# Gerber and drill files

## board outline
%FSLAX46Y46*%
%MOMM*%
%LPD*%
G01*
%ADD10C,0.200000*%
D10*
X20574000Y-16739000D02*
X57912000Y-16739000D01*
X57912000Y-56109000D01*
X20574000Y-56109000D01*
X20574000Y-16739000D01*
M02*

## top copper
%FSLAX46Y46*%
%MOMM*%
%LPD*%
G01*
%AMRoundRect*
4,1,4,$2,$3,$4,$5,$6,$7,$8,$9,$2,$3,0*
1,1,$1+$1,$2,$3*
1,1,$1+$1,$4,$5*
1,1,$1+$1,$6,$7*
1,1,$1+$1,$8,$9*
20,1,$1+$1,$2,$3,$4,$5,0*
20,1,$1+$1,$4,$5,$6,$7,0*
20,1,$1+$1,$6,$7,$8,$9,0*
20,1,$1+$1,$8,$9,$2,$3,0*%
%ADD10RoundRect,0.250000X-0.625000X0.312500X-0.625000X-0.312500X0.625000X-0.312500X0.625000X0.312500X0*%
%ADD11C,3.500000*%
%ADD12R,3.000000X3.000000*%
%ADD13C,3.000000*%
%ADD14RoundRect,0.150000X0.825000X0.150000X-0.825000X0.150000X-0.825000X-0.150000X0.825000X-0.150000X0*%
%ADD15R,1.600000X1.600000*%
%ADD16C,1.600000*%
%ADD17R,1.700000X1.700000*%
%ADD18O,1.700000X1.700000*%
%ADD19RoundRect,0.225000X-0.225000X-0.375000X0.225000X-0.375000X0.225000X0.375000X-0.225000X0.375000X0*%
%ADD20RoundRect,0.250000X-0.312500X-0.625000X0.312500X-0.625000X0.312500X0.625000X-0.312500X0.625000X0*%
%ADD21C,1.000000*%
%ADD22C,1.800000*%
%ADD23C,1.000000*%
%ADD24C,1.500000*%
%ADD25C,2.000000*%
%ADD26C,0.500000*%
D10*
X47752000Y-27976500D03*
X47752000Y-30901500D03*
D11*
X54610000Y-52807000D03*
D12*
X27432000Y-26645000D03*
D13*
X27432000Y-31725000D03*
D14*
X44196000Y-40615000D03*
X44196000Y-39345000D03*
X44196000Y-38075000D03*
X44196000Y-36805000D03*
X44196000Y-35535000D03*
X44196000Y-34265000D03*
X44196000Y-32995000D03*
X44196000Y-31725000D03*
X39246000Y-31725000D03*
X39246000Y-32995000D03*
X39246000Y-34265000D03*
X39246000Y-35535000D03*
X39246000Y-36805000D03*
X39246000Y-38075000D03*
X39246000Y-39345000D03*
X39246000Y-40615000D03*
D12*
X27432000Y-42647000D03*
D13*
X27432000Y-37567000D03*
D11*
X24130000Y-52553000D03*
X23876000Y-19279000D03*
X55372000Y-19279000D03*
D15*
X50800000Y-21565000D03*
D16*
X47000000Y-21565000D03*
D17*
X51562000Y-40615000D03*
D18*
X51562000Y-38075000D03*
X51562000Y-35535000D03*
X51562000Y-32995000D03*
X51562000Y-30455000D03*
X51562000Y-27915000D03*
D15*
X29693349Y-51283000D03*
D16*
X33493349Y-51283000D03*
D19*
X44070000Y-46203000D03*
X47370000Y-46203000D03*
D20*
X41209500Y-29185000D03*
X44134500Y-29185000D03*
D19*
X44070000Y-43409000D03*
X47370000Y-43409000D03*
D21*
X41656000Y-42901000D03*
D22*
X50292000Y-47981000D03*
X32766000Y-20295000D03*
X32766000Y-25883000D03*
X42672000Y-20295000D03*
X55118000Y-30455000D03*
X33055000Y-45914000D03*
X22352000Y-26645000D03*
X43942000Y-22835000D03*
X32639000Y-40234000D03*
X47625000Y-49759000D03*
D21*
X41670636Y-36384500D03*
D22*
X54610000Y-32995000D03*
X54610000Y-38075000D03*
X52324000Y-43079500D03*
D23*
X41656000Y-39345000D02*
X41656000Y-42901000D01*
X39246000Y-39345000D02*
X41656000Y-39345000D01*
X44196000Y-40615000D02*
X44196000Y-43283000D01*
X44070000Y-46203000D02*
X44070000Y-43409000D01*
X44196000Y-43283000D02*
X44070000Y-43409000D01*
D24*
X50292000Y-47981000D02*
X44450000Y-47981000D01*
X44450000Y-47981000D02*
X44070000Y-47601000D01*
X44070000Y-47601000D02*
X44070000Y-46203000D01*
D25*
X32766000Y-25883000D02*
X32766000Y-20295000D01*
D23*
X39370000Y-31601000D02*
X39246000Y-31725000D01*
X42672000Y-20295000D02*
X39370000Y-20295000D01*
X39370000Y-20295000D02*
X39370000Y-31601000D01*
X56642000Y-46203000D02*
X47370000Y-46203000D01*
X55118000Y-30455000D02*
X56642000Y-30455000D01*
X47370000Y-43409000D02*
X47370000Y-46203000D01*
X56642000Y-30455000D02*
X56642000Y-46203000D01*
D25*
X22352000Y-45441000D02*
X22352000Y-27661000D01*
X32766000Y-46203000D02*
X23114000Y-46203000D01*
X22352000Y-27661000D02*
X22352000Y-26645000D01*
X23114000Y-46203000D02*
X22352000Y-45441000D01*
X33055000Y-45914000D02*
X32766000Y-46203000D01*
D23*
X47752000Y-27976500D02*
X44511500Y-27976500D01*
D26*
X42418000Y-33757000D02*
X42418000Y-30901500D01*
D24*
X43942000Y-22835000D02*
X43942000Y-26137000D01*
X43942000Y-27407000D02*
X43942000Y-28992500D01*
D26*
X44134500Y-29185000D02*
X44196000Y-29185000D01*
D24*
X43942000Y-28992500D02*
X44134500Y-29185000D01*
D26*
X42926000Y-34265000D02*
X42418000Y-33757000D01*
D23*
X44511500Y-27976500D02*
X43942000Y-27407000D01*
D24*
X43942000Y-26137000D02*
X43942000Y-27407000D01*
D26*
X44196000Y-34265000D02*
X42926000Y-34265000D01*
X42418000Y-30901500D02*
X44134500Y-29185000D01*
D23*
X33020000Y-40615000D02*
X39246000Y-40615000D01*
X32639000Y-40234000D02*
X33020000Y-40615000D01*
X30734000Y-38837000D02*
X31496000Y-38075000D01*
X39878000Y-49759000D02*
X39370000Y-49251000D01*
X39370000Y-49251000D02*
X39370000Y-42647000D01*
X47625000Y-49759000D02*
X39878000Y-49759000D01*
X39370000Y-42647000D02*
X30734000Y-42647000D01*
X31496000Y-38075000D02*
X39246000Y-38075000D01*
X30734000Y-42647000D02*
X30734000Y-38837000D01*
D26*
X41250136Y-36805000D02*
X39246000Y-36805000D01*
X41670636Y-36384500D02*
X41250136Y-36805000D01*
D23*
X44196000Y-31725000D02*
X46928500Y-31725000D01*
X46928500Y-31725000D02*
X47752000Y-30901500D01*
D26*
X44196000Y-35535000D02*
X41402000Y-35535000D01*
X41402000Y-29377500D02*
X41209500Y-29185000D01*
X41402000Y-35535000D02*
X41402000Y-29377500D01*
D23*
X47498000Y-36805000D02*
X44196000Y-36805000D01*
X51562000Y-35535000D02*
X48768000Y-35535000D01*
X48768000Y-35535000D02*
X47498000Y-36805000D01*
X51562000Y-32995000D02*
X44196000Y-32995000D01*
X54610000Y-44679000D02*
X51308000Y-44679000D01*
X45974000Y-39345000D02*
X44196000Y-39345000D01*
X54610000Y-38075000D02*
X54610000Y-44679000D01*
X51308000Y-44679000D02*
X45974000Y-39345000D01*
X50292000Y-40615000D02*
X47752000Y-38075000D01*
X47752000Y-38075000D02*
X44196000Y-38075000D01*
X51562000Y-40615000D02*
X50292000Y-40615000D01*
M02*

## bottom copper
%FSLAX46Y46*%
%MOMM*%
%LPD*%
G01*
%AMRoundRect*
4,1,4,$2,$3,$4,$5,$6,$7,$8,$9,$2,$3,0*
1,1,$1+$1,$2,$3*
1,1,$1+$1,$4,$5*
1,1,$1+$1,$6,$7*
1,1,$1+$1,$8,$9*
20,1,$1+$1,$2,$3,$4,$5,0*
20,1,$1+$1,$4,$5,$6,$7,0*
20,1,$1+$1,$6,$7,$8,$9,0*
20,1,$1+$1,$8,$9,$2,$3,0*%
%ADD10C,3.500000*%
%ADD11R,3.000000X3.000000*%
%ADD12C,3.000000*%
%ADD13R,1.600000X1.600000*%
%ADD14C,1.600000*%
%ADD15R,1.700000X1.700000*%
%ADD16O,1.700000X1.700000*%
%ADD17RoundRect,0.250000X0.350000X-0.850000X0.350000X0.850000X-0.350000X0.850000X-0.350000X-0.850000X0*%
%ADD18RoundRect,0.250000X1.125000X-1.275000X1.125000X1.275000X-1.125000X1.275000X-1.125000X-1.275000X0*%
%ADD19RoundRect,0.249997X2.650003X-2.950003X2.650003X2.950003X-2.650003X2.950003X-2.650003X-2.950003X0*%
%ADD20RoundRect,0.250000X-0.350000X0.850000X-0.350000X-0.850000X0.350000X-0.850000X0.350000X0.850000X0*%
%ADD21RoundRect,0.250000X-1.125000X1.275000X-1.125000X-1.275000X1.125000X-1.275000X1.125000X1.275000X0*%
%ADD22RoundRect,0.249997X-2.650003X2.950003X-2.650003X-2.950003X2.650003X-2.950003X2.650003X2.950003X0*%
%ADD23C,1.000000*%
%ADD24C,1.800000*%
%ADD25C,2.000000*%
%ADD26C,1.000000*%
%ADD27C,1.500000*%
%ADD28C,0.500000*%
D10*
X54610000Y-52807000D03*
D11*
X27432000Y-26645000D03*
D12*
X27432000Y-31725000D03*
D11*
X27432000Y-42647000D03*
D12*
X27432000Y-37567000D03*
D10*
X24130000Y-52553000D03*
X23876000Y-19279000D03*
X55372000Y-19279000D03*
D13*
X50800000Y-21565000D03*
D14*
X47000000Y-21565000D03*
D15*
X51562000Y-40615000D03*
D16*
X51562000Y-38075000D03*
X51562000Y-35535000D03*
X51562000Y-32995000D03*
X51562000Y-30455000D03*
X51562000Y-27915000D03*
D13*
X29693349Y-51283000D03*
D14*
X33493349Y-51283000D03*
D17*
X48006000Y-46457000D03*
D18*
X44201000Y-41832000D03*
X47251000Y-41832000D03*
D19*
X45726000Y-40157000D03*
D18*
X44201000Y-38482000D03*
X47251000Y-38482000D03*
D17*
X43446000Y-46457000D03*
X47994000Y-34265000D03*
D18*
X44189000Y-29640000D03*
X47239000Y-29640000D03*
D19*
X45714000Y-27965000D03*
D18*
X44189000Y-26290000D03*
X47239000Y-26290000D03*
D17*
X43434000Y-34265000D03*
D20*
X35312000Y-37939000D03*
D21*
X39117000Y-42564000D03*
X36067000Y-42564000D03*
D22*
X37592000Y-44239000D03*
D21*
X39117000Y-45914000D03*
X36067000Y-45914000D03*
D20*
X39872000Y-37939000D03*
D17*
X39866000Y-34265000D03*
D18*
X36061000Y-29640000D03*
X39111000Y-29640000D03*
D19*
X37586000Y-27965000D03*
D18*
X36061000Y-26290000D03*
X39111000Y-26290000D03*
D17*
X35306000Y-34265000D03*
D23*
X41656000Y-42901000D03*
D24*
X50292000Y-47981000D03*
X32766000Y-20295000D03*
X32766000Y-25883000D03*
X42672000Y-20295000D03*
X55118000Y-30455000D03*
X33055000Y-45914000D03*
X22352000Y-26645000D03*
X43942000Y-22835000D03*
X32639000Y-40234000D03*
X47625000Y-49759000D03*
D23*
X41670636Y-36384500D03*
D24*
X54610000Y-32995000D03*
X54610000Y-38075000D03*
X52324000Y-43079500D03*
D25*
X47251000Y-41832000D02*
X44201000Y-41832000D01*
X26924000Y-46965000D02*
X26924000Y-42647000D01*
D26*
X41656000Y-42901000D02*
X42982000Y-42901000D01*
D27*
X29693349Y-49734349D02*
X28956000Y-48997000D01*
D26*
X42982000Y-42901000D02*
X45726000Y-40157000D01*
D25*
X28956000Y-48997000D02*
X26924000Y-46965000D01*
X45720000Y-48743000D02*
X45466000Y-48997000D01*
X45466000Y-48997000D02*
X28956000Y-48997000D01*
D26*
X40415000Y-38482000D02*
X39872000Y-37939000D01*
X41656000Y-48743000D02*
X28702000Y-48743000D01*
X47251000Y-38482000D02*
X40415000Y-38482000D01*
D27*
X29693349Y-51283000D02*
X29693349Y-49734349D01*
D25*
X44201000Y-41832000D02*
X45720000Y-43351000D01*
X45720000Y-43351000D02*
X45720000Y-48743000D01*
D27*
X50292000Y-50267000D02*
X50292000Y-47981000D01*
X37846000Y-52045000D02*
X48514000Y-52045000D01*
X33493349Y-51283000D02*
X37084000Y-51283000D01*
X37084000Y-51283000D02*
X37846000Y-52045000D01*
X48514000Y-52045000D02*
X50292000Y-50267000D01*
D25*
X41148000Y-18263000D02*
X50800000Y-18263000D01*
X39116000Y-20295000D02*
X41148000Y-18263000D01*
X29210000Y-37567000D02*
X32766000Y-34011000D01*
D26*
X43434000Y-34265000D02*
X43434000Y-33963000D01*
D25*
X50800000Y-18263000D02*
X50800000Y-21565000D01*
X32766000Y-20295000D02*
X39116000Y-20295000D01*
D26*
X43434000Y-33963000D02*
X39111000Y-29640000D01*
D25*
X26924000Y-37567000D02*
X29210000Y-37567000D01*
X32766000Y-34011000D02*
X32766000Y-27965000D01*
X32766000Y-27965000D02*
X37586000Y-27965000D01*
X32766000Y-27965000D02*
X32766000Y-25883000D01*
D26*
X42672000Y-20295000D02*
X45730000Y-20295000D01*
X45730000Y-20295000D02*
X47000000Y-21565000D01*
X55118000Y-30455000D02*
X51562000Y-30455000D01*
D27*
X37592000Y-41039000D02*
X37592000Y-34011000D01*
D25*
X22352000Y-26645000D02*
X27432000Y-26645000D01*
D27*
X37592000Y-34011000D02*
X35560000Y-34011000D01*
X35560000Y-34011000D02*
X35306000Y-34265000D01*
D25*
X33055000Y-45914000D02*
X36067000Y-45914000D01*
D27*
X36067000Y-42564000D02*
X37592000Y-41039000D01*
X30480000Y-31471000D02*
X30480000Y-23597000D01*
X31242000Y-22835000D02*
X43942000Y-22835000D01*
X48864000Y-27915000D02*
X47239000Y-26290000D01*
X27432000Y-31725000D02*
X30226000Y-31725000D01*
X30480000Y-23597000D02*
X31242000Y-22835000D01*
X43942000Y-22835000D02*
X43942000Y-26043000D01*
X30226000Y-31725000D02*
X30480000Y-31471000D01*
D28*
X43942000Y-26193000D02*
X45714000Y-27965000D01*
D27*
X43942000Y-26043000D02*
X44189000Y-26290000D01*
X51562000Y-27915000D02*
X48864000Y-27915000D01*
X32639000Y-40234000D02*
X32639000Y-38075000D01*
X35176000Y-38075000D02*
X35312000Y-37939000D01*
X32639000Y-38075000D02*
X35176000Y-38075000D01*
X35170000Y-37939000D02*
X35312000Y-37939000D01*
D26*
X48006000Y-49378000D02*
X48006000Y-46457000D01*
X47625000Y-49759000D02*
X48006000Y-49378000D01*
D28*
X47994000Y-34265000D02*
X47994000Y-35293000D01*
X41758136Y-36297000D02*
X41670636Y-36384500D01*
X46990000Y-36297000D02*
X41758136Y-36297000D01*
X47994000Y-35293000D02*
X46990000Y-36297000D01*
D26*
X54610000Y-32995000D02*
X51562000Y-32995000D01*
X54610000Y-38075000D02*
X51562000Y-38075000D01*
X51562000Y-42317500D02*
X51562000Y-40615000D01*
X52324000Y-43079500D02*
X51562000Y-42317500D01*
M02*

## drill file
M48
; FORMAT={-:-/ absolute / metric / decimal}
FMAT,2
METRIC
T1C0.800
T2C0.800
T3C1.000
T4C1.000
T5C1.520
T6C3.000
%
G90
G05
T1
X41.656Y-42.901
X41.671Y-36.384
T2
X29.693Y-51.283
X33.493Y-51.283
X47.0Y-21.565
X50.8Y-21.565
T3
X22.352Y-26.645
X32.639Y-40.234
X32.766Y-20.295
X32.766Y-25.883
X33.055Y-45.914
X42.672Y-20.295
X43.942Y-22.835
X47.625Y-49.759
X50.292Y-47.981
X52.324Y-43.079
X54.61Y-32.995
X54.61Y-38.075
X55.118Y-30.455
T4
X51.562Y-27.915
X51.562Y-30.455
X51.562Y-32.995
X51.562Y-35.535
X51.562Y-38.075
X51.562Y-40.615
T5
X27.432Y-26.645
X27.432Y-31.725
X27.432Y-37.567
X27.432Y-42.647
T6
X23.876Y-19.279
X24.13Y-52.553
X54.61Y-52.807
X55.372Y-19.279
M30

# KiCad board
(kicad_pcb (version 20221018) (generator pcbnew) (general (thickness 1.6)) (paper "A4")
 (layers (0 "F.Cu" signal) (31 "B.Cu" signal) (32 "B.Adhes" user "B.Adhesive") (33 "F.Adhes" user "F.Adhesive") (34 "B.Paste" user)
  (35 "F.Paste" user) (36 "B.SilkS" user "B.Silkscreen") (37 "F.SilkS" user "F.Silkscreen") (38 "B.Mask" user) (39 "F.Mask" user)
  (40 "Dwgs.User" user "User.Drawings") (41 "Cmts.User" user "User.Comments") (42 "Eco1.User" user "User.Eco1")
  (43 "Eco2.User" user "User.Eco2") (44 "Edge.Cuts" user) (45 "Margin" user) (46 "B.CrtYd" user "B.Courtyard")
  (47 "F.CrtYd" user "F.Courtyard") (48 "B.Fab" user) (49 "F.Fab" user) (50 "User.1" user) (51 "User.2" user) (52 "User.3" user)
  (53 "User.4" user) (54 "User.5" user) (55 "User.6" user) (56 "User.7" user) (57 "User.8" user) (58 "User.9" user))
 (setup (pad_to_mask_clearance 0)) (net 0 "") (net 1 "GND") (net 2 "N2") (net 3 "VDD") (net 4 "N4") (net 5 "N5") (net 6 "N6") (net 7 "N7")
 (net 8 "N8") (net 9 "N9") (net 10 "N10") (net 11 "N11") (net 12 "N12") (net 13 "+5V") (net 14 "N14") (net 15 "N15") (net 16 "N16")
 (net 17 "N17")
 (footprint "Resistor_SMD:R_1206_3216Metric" (layer "F.Cu") (at 47.752 29.439 -90)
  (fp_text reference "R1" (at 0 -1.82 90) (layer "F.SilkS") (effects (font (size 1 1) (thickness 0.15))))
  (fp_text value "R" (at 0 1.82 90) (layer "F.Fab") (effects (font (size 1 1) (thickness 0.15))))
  (pad "1" smd roundrect (at -1.4625 0 270) (size 1.125 1.75) (layers "F.Cu" "F.Paste" "F.Mask") (roundrect_rratio 0.222222) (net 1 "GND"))
  (pad "2" smd roundrect (at 1.4625 0 270) (size 1.125 1.75) (layers "F.Cu" "F.Paste" "F.Mask") (roundrect_rratio 0.222222) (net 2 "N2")))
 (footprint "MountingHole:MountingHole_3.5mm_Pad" (layer "F.Cu") (at 54.61 52.807)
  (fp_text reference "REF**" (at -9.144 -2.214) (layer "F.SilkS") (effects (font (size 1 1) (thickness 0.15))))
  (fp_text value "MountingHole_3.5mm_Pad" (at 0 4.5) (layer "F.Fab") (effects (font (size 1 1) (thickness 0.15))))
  (pad "1" thru_hole circle (at 0 0) (size 3.5 3.5) (drill 3) (layers "*.Cu" "*.Mask")))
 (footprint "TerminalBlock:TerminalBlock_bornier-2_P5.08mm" (layer "F.Cu") (at 27.432 26.645 -90)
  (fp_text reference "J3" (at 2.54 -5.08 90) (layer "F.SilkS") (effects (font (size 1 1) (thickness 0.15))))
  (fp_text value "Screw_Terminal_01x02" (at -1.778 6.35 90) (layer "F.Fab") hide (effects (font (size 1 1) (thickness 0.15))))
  (pad "1" thru_hole rect (at 0 0 270) (size 3 3) (drill 1.52) (layers "*.Cu" "*.Mask") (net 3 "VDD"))
  (pad "2" thru_hole circle (at 5.08 0 270) (size 3 3) (drill 1.52) (layers "*.Cu" "*.Mask") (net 1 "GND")))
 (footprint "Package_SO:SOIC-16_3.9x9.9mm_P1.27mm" (layer "F.Cu") (at 41.721 36.17 180)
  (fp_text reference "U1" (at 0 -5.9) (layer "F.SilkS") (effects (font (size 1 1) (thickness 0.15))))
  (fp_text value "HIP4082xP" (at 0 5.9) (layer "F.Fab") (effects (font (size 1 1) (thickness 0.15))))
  (pad "1" smd roundrect (at -2.475 -4.445 180) (size 1.95 0.6) (layers "F.Cu" "F.Paste" "F.Mask") (roundrect_rratio 0.25) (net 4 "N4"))
  (pad "2" smd roundrect (at -2.475 -3.175 180) (size 1.95 0.6) (layers "F.Cu" "F.Paste" "F.Mask") (roundrect_rratio 0.25) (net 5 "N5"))
  (pad "3" smd roundrect (at -2.475 -1.905 180) (size 1.95 0.6) (layers "F.Cu" "F.Paste" "F.Mask") (roundrect_rratio 0.25) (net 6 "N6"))
  (pad "4" smd roundrect (at -2.475 -0.635 180) (size 1.95 0.6) (layers "F.Cu" "F.Paste" "F.Mask") (roundrect_rratio 0.25) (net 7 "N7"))
  (pad "5" smd roundrect (at -2.475 0.635 180) (size 1.95 0.6) (layers "F.Cu" "F.Paste" "F.Mask") (roundrect_rratio 0.25) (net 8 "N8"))
  (pad "6" smd roundrect (at -2.475 1.905 180) (size 1.95 0.6) (layers "F.Cu" "F.Paste" "F.Mask") (roundrect_rratio 0.25) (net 1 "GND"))
  (pad "7" smd roundrect (at -2.475 3.175 180) (size 1.95 0.6) (layers "F.Cu" "F.Paste" "F.Mask") (roundrect_rratio 0.25) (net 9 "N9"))
  (pad "8" smd roundrect (at -2.475 4.445 180) (size 1.95 0.6) (layers "F.Cu" "F.Paste" "F.Mask") (roundrect_rratio 0.25) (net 2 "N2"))
  (pad "9" smd roundrect (at 2.475 4.445 180) (size 1.95 0.6) (layers "F.Cu" "F.Paste" "F.Mask") (roundrect_rratio 0.25) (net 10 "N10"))
  (pad "10" smd roundrect (at 2.475 3.175 180) (size 1.95 0.6) (layers "F.Cu" "F.Paste" "F.Mask") (roundrect_rratio 0.25) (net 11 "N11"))
  (pad "11" smd roundrect (at 2.475 1.905 180) (size 1.95 0.6) (layers "F.Cu" "F.Paste" "F.Mask") (roundrect_rratio 0.25) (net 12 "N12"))
  (pad "12" smd roundrect (at 2.475 0.635 180) (size 1.95 0.6) (layers "F.Cu" "F.Paste" "F.Mask") (roundrect_rratio 0.25) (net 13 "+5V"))
  (pad "13" smd roundrect (at 2.475 -0.635 180) (size 1.95 0.6) (layers "F.Cu" "F.Paste" "F.Mask") (roundrect_rratio 0.25) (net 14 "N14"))
  (pad "14" smd roundrect (at 2.475 -1.905 180) (size 1.95 0.6) (layers "F.Cu" "F.Paste" "F.Mask") (roundrect_rratio 0.25) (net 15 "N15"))
  (pad "15" smd roundrect (at 2.475 -3.175 180) (size 1.95 0.6) (layers "F.Cu" "F.Paste" "F.Mask") (roundrect_rratio 0.25) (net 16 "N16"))
  (pad "16" smd roundrect (at 2.475 -4.445 180) (size 1.95 0.6) (layers "F.Cu" "F.Paste" "F.Mask") (roundrect_rratio 0.25) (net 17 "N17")))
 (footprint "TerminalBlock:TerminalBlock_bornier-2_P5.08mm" (layer "F.Cu") (at 27.432 42.647 90)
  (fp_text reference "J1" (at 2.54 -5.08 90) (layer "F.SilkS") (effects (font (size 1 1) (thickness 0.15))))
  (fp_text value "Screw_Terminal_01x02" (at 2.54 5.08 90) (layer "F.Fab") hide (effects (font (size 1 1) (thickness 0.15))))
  (pad "1" thru_hole rect (at 0 0 90) (size 3 3) (drill 1.52) (layers "*.Cu" "*.Mask") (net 16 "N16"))
  (pad "2" thru_hole circle (at 5.08 0 90) (size 3 3) (drill 1.52) (layers "*.Cu" "*.Mask") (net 12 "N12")))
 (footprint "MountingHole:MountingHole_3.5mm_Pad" (layer "F.Cu") (at 24.13 52.553)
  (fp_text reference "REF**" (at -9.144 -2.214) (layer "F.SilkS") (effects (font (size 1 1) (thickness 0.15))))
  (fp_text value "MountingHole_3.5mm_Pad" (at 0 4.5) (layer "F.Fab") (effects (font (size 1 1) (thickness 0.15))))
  (pad "1" thru_hole circle (at 0 0) (size 3.5 3.5) (drill 3) (layers "*.Cu" "*.Mask")))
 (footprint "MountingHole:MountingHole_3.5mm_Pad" (layer "F.Cu") (at 23.876 19.279)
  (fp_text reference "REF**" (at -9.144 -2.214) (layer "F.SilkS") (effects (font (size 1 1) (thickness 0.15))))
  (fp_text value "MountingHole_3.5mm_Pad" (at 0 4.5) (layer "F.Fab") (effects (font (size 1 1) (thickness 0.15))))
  (pad "1" thru_hole circle (at 0 0) (size 3.5 3.5) (drill 3) (layers "*.Cu" "*.Mask")))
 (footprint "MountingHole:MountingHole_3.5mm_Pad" (layer "F.Cu") (at 55.372 19.279)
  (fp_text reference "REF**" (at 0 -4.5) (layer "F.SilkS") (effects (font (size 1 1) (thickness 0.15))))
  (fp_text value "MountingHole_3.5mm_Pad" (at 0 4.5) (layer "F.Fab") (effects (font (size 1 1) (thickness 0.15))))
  (pad "1" thru_hole circle (at 0 0) (size 3.5 3.5) (drill 3) (layers "*.Cu" "*.Mask")))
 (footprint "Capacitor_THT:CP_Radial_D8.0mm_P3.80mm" (layer "F.Cu") (at 50.8 21.565 180)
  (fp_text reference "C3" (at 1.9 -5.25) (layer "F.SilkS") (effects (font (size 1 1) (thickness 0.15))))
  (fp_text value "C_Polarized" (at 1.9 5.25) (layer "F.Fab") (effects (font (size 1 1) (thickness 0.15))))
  (pad "1" thru_hole rect (at 0 0 180) (size 1.6 1.6) (drill 0.8) (layers "*.Cu" "*.Mask") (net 12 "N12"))
  (pad "2" thru_hole circle (at 3.8 0 180) (size 1.6 1.6) (drill 0.8) (layers "*.Cu" "*.Mask") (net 10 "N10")))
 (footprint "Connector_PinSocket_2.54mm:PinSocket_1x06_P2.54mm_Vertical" (layer "F.Cu") (at 51.562 40.615 180)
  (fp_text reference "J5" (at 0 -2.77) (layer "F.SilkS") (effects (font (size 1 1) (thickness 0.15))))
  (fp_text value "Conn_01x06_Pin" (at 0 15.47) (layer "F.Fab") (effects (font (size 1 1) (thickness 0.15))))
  (pad "1" thru_hole rect (at 0 0 180) (size 1.7 1.7) (drill 1) (layers "*.Cu" "*.Mask") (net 6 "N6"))
  (pad "2" thru_hole oval (at 0 2.54 180) (size 1.7 1.7) (drill 1) (layers "*.Cu" "*.Mask") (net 5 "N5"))
  (pad "3" thru_hole oval (at 0 5.08 180) (size 1.7 1.7) (drill 1) (layers "*.Cu" "*.Mask") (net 7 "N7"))
  (pad "4" thru_hole oval (at 0 7.62 180) (size 1.7 1.7) (drill 1) (layers "*.Cu" "*.Mask") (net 9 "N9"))
  (pad "5" thru_hole oval (at 0 10.16 180) (size 1.7 1.7) (drill 1) (layers "*.Cu" "*.Mask") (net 13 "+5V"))
  (pad "6" thru_hole oval (at 0 12.7 180) (size 1.7 1.7) (drill 1) (layers "*.Cu" "*.Mask") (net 1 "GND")))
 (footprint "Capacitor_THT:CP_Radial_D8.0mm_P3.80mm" (layer "F.Cu") (at 29.693349 51.283)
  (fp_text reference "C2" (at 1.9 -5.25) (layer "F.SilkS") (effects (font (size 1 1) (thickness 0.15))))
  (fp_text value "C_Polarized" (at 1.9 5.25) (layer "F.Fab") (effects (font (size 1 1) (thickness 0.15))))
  (pad "1" thru_hole rect (at 0 0) (size 1.6 1.6) (drill 0.8) (layers "*.Cu" "*.Mask") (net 16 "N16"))
  (pad "2" thru_hole circle (at 3.8 0) (size 1.6 1.6) (drill 0.8) (layers "*.Cu" "*.Mask") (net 4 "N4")))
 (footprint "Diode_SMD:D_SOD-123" (layer "F.Cu") (at 45.72 46.203)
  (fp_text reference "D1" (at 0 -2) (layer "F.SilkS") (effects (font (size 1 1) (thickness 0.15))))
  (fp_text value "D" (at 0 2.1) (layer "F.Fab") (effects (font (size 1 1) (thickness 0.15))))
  (pad "1" smd roundrect (at -1.65 0) (size 0.9 1.2) (layers "F.Cu" "F.Paste" "F.Mask") (roundrect_rratio 0.25) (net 4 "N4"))
  (pad "2" smd roundrect (at 1.65 0) (size 0.9 1.2) (layers "F.Cu" "F.Paste" "F.Mask") (roundrect_rratio 0.25) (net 13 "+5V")))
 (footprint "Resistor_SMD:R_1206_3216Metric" (layer "F.Cu") (at 42.672 29.185)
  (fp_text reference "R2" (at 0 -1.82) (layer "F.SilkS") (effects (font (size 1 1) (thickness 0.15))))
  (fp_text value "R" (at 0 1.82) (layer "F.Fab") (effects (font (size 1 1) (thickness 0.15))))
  (pad "1" smd roundrect (at -1.4625 0) (size 1.125 1.75) (layers "F.Cu" "F.Paste" "F.Mask") (roundrect_rratio 0.222222) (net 8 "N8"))
  (pad "2" smd roundrect (at 1.4625 0) (size 1.125 1.75) (layers "F.Cu" "F.Paste" "F.Mask") (roundrect_rratio 0.222222) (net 1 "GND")))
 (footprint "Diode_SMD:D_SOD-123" (layer "F.Cu") (at 45.72 43.409)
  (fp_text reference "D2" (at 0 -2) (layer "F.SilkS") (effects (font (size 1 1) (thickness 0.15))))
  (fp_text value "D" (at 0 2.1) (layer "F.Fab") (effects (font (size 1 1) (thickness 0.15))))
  (pad "1" smd roundrect (at -1.65 0) (size 0.9 1.2) (layers "F.Cu" "F.Paste" "F.Mask") (roundrect_rratio 0.25) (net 4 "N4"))
  (pad "2" smd roundrect (at 1.65 0) (size 0.9 1.2) (layers "F.Cu" "F.Paste" "F.Mask") (roundrect_rratio 0.25) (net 13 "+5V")))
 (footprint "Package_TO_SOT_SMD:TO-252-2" (layer "B.Cu") (at 45.726 41.417 90)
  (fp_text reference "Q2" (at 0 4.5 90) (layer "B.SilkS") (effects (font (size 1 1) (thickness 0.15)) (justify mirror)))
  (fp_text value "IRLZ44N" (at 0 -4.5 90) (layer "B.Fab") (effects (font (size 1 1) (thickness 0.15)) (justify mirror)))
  (pad "1" smd roundrect (at -5.04 2.28 90) (size 2.2 1.2) (layers "B.Cu" "B.Paste" "B.Mask") (roundrect_rratio 0.208333) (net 15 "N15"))
  (pad "2" smd roundrect (at -0.415 -1.525 90) (size 3.05 2.75) (layers "B.Cu" "B.Paste") (roundrect_rratio 0.090909) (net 16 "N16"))
  (pad "2" smd roundrect (at -0.415 1.525 90) (size 3.05 2.75) (layers "B.Cu" "B.Paste") (roundrect_rratio 0.090909) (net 16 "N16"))
  (pad "2" smd roundrect (at 1.26 0 90) (size 6.4 5.8) (layers "B.Cu" "B.Mask") (roundrect_rratio 0.043103) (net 16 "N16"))
  (pad "2" smd roundrect (at 2.935 -1.525 90) (size 3.05 2.75) (layers "B.Cu" "B.Paste") (roundrect_rratio 0.090909) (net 16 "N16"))
  (pad "2" smd roundrect (at 2.935 1.525 90) (size 3.05 2.75) (layers "B.Cu" "B.Paste") (roundrect_rratio 0.090909) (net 16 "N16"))
  (pad "3" smd roundrect (at -5.04 -2.28 90) (size 2.2 1.2) (layers "B.Cu" "B.Paste" "B.Mask") (roundrect_rratio 0.208333) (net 1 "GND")))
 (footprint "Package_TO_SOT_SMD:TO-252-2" (layer "B.Cu") (at 45.714 29.225 90)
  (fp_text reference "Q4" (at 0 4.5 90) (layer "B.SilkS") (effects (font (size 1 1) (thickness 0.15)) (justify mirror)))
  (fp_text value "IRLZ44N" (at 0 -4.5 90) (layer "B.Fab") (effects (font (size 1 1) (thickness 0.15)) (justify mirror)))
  (pad "1" smd roundrect (at -5.04 2.28 90) (size 2.2 1.2) (layers "B.Cu" "B.Paste" "B.Mask") (roundrect_rratio 0.208333) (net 14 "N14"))
  (pad "2" smd roundrect (at -0.415 -1.525 90) (size 3.05 2.75) (layers "B.Cu" "B.Paste") (roundrect_rratio 0.090909) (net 1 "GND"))
  (pad "2" smd roundrect (at -0.415 1.525 90) (size 3.05 2.75) (layers "B.Cu" "B.Paste") (roundrect_rratio 0.090909) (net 1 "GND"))
  (pad "2" smd roundrect (at 1.26 0 90) (size 6.4 5.8) (layers "B.Cu" "B.Mask") (roundrect_rratio 0.043103) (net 1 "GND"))
  (pad "2" smd roundrect (at 2.935 -1.525 90) (size 3.05 2.75) (layers "B.Cu" "B.Paste") (roundrect_rratio 0.090909) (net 1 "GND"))
  (pad "2" smd roundrect (at 2.935 1.525 90) (size 3.05 2.75) (layers "B.Cu" "B.Paste") (roundrect_rratio 0.090909) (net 1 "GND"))
  (pad "3" smd roundrect (at -5.04 -2.28 90) (size 2.2 1.2) (layers "B.Cu" "B.Paste" "B.Mask") (roundrect_rratio 0.208333) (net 12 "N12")))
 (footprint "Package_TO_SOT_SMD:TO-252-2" (layer "B.Cu") (at 37.592 42.979 -90)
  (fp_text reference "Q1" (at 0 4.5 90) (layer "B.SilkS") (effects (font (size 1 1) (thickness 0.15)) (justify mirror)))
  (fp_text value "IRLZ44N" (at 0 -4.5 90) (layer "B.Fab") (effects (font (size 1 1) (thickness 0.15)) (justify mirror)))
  (pad "1" smd roundrect (at -5.04 2.28 270) (size 2.2 1.2) (layers "B.Cu" "B.Paste" "B.Mask") (roundrect_rratio 0.208333) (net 17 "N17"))
  (pad "2" smd roundrect (at -0.415 -1.525 270) (size 3.05 2.75) (layers "B.Cu" "B.Paste") (roundrect_rratio 0.090909) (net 3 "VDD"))
  (pad "2" smd roundrect (at -0.415 1.525 270) (size 3.05 2.75) (layers "B.Cu" "B.Paste") (roundrect_rratio 0.090909) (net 3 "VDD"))
  (pad "2" smd roundrect (at 1.26 0 270) (size 6.4 5.8) (layers "B.Cu" "B.Mask") (roundrect_rratio 0.043103) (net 3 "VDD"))
  (pad "2" smd roundrect (at 2.935 -1.525 270) (size 3.05 2.75) (layers "B.Cu" "B.Paste") (roundrect_rratio 0.090909) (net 3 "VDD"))
  (pad "2" smd roundrect (at 2.935 1.525 270) (size 3.05 2.75) (layers "B.Cu" "B.Paste") (roundrect_rratio 0.090909) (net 3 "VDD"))
  (pad "3" smd roundrect (at -5.04 -2.28 270) (size 2.2 1.2) (layers "B.Cu" "B.Paste" "B.Mask") (roundrect_rratio 0.208333) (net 16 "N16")))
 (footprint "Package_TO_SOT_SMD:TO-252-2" (layer "B.Cu") (at 37.586 29.225 90)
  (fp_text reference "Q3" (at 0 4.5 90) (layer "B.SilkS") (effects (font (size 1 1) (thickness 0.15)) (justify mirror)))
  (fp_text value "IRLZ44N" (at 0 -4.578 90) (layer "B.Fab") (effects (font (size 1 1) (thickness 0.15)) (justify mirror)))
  (pad "1" smd roundrect (at -5.04 2.28 90) (size 2.2 1.2) (layers "B.Cu" "B.Paste" "B.Mask") (roundrect_rratio 0.208333) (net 11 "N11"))
  (pad "2" smd roundrect (at -0.415 -1.525 90) (size 3.05 2.75) (layers "B.Cu" "B.Paste") (roundrect_rratio 0.090909) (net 12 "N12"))
  (pad "2" smd roundrect (at -0.415 1.525 90) (size 3.05 2.75) (layers "B.Cu" "B.Paste") (roundrect_rratio 0.090909) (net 12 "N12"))
  (pad "2" smd roundrect (at 1.26 0 90) (size 6.4 5.8) (layers "B.Cu" "B.Mask") (roundrect_rratio 0.043103) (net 12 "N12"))
  (pad "2" smd roundrect (at 2.935 -1.525 90) (size 3.05 2.75) (layers "B.Cu" "B.Paste") (roundrect_rratio 0.090909) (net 12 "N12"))
  (pad "2" smd roundrect (at 2.935 1.525 90) (size 3.05 2.75) (layers "B.Cu" "B.Paste") (roundrect_rratio 0.090909) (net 12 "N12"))
  (pad "3" smd roundrect (at -5.04 -2.28 90) (size 2.2 1.2) (layers "B.Cu" "B.Paste" "B.Mask") (roundrect_rratio 0.208333) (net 3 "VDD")))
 (gr_rect (start 20.574 16.739) (end 57.912 56.109) (stroke (width 0.2) (type default)) (fill none) (layer "Edge.Cuts"))
 (segment (start 41.656 39.345) (end 41.656 42.901) (width 1) (layer "F.Cu") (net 16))
 (segment (start 39.246 39.345) (end 41.656 39.345) (width 1) (layer "F.Cu") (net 16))
 (via (at 41.656 42.901) (size 1) (drill 0.8) (layers "F.Cu" "B.Cu") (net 16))
 (segment (start 47.251 41.832) (end 44.201 41.832) (width 2) (layer "B.Cu") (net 16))
 (segment (start 26.924 46.965) (end 26.924 42.647) (width 2) (layer "B.Cu") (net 16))
 (segment (start 41.656 42.901) (end 42.982 42.901) (width 1) (layer "B.Cu") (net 16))
 (segment (start 29.693349 49.734349) (end 28.956 48.997) (width 1.5) (layer "B.Cu") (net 16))
 (segment (start 42.982 42.901) (end 45.726 40.157) (width 1) (layer "B.Cu") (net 16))
 (segment (start 28.956 48.997) (end 26.924 46.965) (width 2) (layer "B.Cu") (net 16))
 (segment (start 45.72 48.743) (end 45.466 48.997) (width 2) (layer "B.Cu") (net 16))
 (segment (start 45.466 48.997) (end 28.956 48.997) (width 2) (layer "B.Cu") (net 16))
 (segment (start 40.415 38.482) (end 39.872 37.939) (width 1) (layer "B.Cu") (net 16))
 (segment (start 41.656 48.743) (end 28.702 48.743) (width 1) (layer "B.Cu") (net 16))
 (segment (start 47.251 38.482) (end 40.415 38.482) (width 1) (layer "B.Cu") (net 16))
 (segment (start 29.693349 51.283) (end 29.693349 49.734349) (width 1.5) (layer "B.Cu") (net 16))
 (segment (start 44.201 41.832) (end 45.72 43.351) (width 2) (layer "B.Cu") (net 16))
 (segment (start 45.72 43.351) (end 45.72 48.743) (width 2) (layer "B.Cu") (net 16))
 (segment (start 44.196 40.615) (end 44.196 43.283) (width 1) (layer "F.Cu") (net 4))
 (segment (start 44.07 46.203) (end 44.07 43.409) (width 1) (layer "F.Cu") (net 4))
 (segment (start 44.196 43.283) (end 44.07 43.409) (width 1) (layer "F.Cu") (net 4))
 (segment (start 50.292 47.981) (end 44.45 47.981) (width 1.5) (layer "F.Cu") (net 4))
 (segment (start 44.45 47.981) (end 44.07 47.601) (width 1.5) (layer "F.Cu") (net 4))
 (segment (start 44.07 47.601) (end 44.07 46.203) (width 1.5) (layer "F.Cu") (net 4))
 (via (at 50.292 47.981) (size 1.8) (drill 1) (layers "F.Cu" "B.Cu") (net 4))
 (segment (start 50.292 50.267) (end 50.292 47.981) (width 1.5) (layer "B.Cu") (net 4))
 (segment (start 37.846 52.045) (end 48.514 52.045) (width 1.5) (layer "B.Cu") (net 4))
 (segment (start 33.493349 51.283) (end 37.084 51.283) (width 1.5) (layer "B.Cu") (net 4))
 (segment (start 37.084 51.283) (end 37.846 52.045) (width 1.5) (layer "B.Cu") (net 4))
 (segment (start 48.514 52.045) (end 50.292 50.267) (width 1.5) (layer "B.Cu") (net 4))
 (segment (start 32.766 25.883) (end 32.766 20.295) (width 2) (layer "F.Cu") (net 12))
 (via (at 32.766 20.295) (size 1.8) (drill 1) (layers "F.Cu" "B.Cu") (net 12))
 (via (at 32.766 25.883) (size 1.8) (drill 1) (layers "F.Cu" "B.Cu") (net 12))
 (segment (start 41.148 18.263) (end 50.8 18.263) (width 2) (layer "B.Cu") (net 12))
 (segment (start 39.116 20.295) (end 41.148 18.263) (width 2) (layer "B.Cu") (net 12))
 (segment (start 29.21 37.567) (end 32.766 34.011) (width 2) (layer "B.Cu") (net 12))
 (segment (start 43.434 34.265) (end 43.434 33.963) (width 1) (layer "B.Cu") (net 12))
 (segment (start 50.8 18.263) (end 50.8 21.565) (width 2) (layer "B.Cu") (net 12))
 (segment (start 32.766 20.295) (end 39.116 20.295) (width 2) (layer "B.Cu") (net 12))
 (segment (start 43.434 33.963) (end 39.111 29.64) (width 1) (layer "B.Cu") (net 12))
 (segment (start 26.924 37.567) (end 29.21 37.567) (width 2) (layer "B.Cu") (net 12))
 (segment (start 32.766 34.011) (end 32.766 27.965) (width 2) (layer "B.Cu") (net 12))
 (segment (start 32.766 27.965) (end 37.586 27.965) (width 2) (layer "B.Cu") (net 12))
 (segment (start 32.766 27.965) (end 32.766 25.883) (width 2) (layer "B.Cu") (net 12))
 (segment (start 39.37 31.601) (end 39.246 31.725) (width 1) (layer "F.Cu") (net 10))
 (segment (start 42.672 20.295) (end 39.37 20.295) (width 1) (layer "F.Cu") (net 10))
 (segment (start 39.37 20.295) (end 39.37 31.601) (width 1) (layer "F.Cu") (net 10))
 (via (at 42.672 20.295) (size 1.8) (drill 1) (layers "F.Cu" "B.Cu") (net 10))
 (segment (start 42.672 20.295) (end 45.73 20.295) (width 1) (layer "B.Cu") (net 10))
 (segment (start 45.73 20.295) (end 47 21.565) (width 1) (layer "B.Cu") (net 10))
 (segment (start 56.642 46.203) (end 47.37 46.203) (width 1) (layer "F.Cu") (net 13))
 (segment (start 55.118 30.455) (end 56.642 30.455) (width 1) (layer "F.Cu") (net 13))
 (segment (start 47.37 43.409) (end 47.37 46.203) (width 1) (layer "F.Cu") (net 13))
 (segment (start 56.642 30.455) (end 56.642 46.203) (width 1) (layer "F.Cu") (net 13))
 (via (at 55.118 30.455) (size 1.8) (drill 1) (layers "F.Cu" "B.Cu") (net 13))
 (segment (start 55.118 30.455) (end 51.562 30.455) (width 1) (layer "B.Cu") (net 13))
 (segment (start 22.352 45.441) (end 22.352 27.661) (width 2) (layer "F.Cu") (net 3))
 (segment (start 32.766 46.203) (end 23.114 46.203) (width 2) (layer "F.Cu") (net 3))
 (segment (start 22.352 27.661) (end 22.352 26.645) (width 2) (layer "F.Cu") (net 3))
 (segment (start 23.114 46.203) (end 22.352 45.441) (width 2) (layer "F.Cu") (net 3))
 (segment (start 33.055 45.914) (end 32.766 46.203) (width 2) (layer "F.Cu") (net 3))
 (via (at 33.055 45.914) (size 1.8) (drill 1) (layers "F.Cu" "B.Cu") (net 3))
 (via (at 22.352 26.645) (size 1.8) (drill 1) (layers "F.Cu" "B.Cu") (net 3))
 (segment (start 37.592 41.039) (end 37.592 34.011) (width 1.5) (layer "B.Cu") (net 3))
 (segment (start 22.352 26.645) (end 27.432 26.645) (width 2) (layer "B.Cu") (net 3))
 (segment (start 37.592 34.011) (end 35.56 34.011) (width 1.5) (layer "B.Cu") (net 3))
 (segment (start 35.56 34.011) (end 35.306 34.265) (width 1.5) (layer "B.Cu") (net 3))
 (segment (start 33.055 45.914) (end 36.067 45.914) (width 2) (layer "B.Cu") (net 3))
 (segment (start 36.067 42.564) (end 37.592 41.039) (width 1.5) (layer "B.Cu") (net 3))
 (segment (start 47.752 27.9765) (end 44.5115 27.9765) (width 1) (layer "F.Cu") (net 1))
 (segment (start 42.418 33.757) (end 42.418 30.9015) (width 0.5) (layer "F.Cu") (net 1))
 (segment (start 43.942 22.835) (end 43.942 26.137) (width 1.5) (layer "F.Cu") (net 1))
 (segment (start 43.942 27.407) (end 43.942 28.9925) (width 1.5) (layer "F.Cu") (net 1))
 (segment (start 44.1345 29.185) (end 44.196 29.185) (width 0.5) (layer "F.Cu") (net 1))
 (segment (start 43.942 28.9925) (end 44.1345 29.185) (width 1.5) (layer "F.Cu") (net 1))
 (segment (start 42.926 34.265) (end 42.418 33.757) (width 0.5) (layer "F.Cu") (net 1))
 (segment (start 44.5115 27.9765) (end 43.942 27.407) (width 1) (layer "F.Cu") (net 1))
 (segment (start 43.942 26.137) (end 43.942 27.407) (width 1.5) (layer "F.Cu") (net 1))
 (segment (start 44.196 34.265) (end 42.926 34.265) (width 0.5) (layer "F.Cu") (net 1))
 (segment (start 42.418 30.9015) (end 44.1345 29.185) (width 0.5) (layer "F.Cu") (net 1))
 (via (at 43.942 22.835) (size 1.8) (drill 1) (layers "F.Cu" "B.Cu") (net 1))
 (segment (start 30.48 31.471) (end 30.48 23.597) (width 1.5) (layer "B.Cu") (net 1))
 (segment (start 31.242 22.835) (end 43.942 22.835) (width 1.5) (layer "B.Cu") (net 1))
 (segment (start 48.864 27.915) (end 47.239 26.29) (width 1.5) (layer "B.Cu") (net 1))
 (segment (start 27.432 31.725) (end 30.226 31.725) (width 1.5) (layer "B.Cu") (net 1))
 (segment (start 30.48 23.597) (end 31.242 22.835) (width 1.5) (layer "B.Cu") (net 1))
 (segment (start 43.942 22.835) (end 43.942 26.043) (width 1.5) (layer "B.Cu") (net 1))
 (segment (start 30.226 31.725) (end 30.48 31.471) (width 1.5) (layer "B.Cu") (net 1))
 (segment (start 43.942 26.193) (end 45.714 27.965) (width 0.5) (layer "B.Cu") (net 1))
 (segment (start 43.942 26.043) (end 44.189 26.29) (width 1.5) (layer "B.Cu") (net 1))
 (segment (start 51.562 27.915) (end 48.864 27.915) (width 1.5) (layer "B.Cu") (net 1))
 (segment (start 33.02 40.615) (end 39.246 40.615) (width 1) (layer "F.Cu") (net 17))
 (segment (start 32.639 40.234) (end 33.02 40.615) (width 1) (layer "F.Cu") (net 17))
 (via (at 32.639 40.234) (size 1.8) (drill 1) (layers "F.Cu" "B.Cu") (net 17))
 (segment (start 32.639 40.234) (end 32.639 38.075) (width 1.5) (layer "B.Cu") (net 17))
 (segment (start 35.176 38.075) (end 35.312 37.939) (width 1.5) (layer "B.Cu") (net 17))
 (segment (start 32.639 38.075) (end 35.176 38.075) (width 1.5) (layer "B.Cu") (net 17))
 (segment (start 35.17 37.939) (end 35.312 37.939) (width 1.5) (layer "B.Cu") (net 17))
 (segment (start 30.734 38.837) (end 31.496 38.075) (width 1) (layer "F.Cu") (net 15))
 (segment (start 39.878 49.759) (end 39.37 49.251) (width 1) (layer "F.Cu") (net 15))
 (segment (start 39.37 49.251) (end 39.37 42.647) (width 1) (layer "F.Cu") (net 15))
 (segment (start 47.625 49.759) (end 39.878 49.759) (width 1) (layer "F.Cu") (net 15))
 (segment (start 39.37 42.647) (end 30.734 42.647) (width 1) (layer "F.Cu") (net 15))
 (segment (start 31.496 38.075) (end 39.246 38.075) (width 1) (layer "F.Cu") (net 15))
 (segment (start 30.734 42.647) (end 30.734 38.837) (width 1) (layer "F.Cu") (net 15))
 (via (at 47.625 49.759) (size 1.8) (drill 1) (layers "F.Cu" "B.Cu") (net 15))
 (segment (start 48.006 49.378) (end 48.006 46.457) (width 1) (layer "B.Cu") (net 15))
 (segment (start 47.625 49.759) (end 48.006 49.378) (width 1) (layer "B.Cu") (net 15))
 (segment (start 41.250136 36.805) (end 39.246 36.805) (width 0.5) (layer "F.Cu") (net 14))
 (segment (start 41.670636 36.3845) (end 41.250136 36.805) (width 0.5) (layer "F.Cu") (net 14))
 (via (at 41.670636 36.3845) (size 1) (drill 0.8) (layers "F.Cu" "B.Cu") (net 14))
 (segment (start 47.994 34.265) (end 47.994 35.293) (width 0.5) (layer "B.Cu") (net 14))
 (segment (start 41.758136 36.297) (end 41.670636 36.3845) (width 0.5) (layer "B.Cu") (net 14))
 (segment (start 46.99 36.297) (end 41.758136 36.297) (width 0.5) (layer "B.Cu") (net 14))
 (segment (start 47.994 35.293) (end 46.99 36.297) (width 0.5) (layer "B.Cu") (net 14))
 (segment (start 44.196 31.725) (end 46.9285 31.725) (width 1) (layer "F.Cu") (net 2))
 (segment (start 46.9285 31.725) (end 47.752 30.9015) (width 1) (layer "F.Cu") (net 2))
 (segment (start 44.196 35.535) (end 41.402 35.535) (width 0.5) (layer "F.Cu") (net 8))
 (segment (start 41.402 29.3775) (end 41.2095 29.185) (width 0.5) (layer "F.Cu") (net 8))
 (segment (start 41.402 35.535) (end 41.402 29.3775) (width 0.5) (layer "F.Cu") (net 8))
 (segment (start 47.498 36.805) (end 44.196 36.805) (width 1) (layer "F.Cu") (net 7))
 (segment (start 51.562 35.535) (end 48.768 35.535) (width 1) (layer "F.Cu") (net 7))
 (segment (start 48.768 35.535) (end 47.498 36.805) (width 1) (layer "F.Cu") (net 7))
 (segment (start 51.562 32.995) (end 44.196 32.995) (width 1) (layer "F.Cu") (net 9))
 (via (at 54.61 32.995) (size 1.8) (drill 1) (layers "F.Cu" "B.Cu") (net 9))
 (segment (start 54.61 32.995) (end 51.562 32.995) (width 1) (layer "B.Cu") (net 9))
 (segment (start 54.61 44.679) (end 51.308 44.679) (width 1) (layer "F.Cu") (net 5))
 (segment (start 45.974 39.345) (end 44.196 39.345) (width 1) (layer "F.Cu") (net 5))
 (segment (start 54.61 38.075) (end 54.61 44.679) (width 1) (layer "F.Cu") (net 5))
 (segment (start 51.308 44.679) (end 45.974 39.345) (width 1) (layer "F.Cu") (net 5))
 (via (at 54.61 38.075) (size 1.8) (drill 1) (layers "F.Cu" "B.Cu") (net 5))
 (segment (start 54.61 38.075) (end 51.562 38.075) (width 1) (layer "B.Cu") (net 5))
 (segment (start 50.292 40.615) (end 47.752 38.075) (width 1) (layer "F.Cu") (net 6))
 (segment (start 47.752 38.075) (end 44.196 38.075) (width 1) (layer "F.Cu") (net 6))
 (segment (start 51.562 40.615) (end 50.292 40.615) (width 1) (layer "F.Cu") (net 6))
 (via (at 52.324 43.0795) (size 1.8) (drill 1) (layers "F.Cu" "B.Cu") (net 6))
 (segment (start 51.562 42.3175) (end 51.562 40.615) (width 1) (layer "B.Cu") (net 6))
 (segment (start 52.324 43.0795) (end 51.562 42.3175) (width 1) (layer "B.Cu") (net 6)))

